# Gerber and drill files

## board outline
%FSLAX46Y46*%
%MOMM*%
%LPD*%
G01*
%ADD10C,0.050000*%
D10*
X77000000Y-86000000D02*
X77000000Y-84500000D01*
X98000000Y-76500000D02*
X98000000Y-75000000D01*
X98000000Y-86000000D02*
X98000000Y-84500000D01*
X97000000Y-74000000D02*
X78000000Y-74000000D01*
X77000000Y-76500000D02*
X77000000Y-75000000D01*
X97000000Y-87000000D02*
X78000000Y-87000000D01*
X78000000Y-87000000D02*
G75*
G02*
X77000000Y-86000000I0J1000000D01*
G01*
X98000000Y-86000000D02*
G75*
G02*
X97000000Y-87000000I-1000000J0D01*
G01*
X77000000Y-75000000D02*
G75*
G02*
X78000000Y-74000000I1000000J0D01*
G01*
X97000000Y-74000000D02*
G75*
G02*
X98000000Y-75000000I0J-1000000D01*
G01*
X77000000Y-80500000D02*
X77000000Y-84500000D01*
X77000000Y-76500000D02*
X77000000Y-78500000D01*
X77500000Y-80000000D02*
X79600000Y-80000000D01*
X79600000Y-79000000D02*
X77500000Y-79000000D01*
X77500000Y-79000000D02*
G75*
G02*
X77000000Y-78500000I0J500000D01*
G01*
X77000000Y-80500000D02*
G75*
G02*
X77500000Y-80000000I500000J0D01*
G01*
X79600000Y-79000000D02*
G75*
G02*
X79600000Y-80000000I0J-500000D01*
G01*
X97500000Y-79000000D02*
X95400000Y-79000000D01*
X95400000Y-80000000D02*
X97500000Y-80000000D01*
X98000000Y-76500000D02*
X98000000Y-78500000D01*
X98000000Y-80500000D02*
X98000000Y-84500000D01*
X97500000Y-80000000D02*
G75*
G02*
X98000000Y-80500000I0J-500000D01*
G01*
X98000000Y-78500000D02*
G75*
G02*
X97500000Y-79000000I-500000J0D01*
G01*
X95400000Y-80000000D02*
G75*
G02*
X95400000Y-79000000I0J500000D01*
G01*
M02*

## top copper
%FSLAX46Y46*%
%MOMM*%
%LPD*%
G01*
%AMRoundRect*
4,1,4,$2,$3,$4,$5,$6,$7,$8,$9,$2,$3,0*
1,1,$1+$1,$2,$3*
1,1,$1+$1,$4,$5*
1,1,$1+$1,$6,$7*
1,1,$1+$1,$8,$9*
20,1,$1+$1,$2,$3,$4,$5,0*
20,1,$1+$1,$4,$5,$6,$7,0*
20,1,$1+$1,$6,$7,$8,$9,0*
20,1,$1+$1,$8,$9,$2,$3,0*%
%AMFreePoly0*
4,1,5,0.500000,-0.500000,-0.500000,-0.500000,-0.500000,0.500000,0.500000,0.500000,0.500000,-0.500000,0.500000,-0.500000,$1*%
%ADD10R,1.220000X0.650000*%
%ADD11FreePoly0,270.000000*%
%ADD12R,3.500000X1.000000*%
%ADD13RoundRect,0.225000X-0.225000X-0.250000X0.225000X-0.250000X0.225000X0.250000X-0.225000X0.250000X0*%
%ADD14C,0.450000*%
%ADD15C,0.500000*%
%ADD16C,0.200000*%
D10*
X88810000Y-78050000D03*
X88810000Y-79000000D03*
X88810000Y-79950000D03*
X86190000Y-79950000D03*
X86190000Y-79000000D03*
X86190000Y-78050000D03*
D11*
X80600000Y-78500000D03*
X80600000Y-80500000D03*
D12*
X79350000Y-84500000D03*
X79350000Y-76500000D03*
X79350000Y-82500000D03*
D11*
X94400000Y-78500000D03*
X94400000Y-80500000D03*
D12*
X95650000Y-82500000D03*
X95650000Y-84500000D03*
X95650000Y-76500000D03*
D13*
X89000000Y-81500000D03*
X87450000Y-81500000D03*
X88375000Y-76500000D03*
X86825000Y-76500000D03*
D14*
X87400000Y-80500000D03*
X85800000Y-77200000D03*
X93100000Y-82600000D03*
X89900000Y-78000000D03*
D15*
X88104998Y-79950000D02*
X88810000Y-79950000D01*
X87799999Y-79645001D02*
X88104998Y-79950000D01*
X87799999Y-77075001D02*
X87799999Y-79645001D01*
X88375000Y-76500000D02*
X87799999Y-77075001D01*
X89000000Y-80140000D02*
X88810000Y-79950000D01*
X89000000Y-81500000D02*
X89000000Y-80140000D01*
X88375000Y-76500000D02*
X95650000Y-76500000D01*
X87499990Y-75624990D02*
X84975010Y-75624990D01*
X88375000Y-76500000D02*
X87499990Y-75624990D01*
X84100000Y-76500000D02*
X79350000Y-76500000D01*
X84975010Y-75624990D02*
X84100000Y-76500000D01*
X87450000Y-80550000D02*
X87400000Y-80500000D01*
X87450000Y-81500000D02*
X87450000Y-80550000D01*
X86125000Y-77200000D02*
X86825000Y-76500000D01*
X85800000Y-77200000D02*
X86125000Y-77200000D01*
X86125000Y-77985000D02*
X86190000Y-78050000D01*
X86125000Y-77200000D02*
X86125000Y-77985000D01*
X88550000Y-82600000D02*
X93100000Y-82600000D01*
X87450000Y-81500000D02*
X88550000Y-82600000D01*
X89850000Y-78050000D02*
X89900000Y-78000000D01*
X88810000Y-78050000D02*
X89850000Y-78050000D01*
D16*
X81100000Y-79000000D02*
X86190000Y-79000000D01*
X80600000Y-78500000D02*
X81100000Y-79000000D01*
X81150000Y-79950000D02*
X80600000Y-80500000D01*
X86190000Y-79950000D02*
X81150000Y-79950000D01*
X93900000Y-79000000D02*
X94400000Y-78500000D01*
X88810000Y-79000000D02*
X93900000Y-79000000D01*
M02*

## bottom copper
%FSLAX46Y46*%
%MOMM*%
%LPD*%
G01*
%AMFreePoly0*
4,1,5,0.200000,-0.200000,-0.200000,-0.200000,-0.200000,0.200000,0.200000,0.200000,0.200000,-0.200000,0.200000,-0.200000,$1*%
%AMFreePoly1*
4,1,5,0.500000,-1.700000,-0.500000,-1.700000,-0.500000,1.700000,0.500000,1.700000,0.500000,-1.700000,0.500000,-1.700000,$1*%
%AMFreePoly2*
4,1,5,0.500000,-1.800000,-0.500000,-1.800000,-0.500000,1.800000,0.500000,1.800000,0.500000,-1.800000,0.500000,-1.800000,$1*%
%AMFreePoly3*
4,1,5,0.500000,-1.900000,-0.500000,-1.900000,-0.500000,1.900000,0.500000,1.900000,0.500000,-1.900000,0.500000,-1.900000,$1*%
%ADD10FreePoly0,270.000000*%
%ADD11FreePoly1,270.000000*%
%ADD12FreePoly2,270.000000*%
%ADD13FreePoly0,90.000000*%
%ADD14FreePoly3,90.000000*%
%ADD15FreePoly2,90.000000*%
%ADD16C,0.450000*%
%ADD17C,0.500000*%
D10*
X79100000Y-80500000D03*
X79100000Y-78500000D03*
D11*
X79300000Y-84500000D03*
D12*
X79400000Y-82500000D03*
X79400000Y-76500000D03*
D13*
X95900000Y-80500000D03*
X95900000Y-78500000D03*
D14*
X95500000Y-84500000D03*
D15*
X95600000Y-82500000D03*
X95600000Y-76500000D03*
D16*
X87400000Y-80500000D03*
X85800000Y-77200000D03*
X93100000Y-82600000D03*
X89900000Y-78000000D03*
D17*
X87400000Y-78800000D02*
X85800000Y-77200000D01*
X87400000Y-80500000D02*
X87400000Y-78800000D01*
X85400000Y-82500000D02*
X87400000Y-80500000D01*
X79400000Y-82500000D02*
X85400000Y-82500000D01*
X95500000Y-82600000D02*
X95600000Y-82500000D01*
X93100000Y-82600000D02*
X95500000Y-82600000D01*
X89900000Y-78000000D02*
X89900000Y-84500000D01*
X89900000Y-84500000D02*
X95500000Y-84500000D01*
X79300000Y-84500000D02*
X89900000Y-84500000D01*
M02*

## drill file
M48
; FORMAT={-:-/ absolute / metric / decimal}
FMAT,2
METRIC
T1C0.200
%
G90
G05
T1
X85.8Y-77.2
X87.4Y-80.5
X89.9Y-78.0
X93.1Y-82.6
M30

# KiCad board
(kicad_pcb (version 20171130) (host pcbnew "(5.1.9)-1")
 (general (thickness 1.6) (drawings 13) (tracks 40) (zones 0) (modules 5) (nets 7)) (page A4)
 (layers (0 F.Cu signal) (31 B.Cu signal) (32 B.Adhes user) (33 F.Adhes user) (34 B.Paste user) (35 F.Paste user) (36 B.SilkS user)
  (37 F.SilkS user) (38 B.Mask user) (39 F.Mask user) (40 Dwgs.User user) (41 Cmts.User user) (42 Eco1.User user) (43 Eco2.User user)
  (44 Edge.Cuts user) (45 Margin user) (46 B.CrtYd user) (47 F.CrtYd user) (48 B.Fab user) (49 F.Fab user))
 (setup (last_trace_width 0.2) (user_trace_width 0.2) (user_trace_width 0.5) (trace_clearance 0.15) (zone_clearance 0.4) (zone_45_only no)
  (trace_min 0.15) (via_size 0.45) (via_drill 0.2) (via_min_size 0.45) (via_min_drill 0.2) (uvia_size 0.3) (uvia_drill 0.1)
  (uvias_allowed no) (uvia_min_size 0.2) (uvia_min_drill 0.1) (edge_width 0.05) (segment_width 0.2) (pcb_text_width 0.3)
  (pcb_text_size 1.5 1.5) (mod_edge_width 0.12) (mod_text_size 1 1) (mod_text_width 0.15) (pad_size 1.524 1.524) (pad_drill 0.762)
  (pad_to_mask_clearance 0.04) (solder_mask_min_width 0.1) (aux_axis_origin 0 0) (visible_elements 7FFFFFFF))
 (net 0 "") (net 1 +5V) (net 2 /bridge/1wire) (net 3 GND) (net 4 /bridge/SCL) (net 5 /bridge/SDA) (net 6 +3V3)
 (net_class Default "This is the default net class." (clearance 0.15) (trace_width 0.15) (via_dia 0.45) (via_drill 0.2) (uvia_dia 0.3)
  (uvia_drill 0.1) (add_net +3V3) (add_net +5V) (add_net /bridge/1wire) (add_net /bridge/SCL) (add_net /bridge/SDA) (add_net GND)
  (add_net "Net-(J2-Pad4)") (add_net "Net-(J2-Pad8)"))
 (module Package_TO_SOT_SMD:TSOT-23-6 (layer F.Cu) (at 87.5 79)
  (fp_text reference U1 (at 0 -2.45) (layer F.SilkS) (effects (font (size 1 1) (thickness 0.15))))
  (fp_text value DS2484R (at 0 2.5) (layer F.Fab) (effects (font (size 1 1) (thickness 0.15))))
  (pad 6 smd rect (at 1.31 -0.95) (size 1.22 0.65) (layers F.Cu F.Paste F.Mask) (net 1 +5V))
  (pad 5 smd rect (at 1.31 0) (size 1.22 0.65) (layers F.Cu F.Paste F.Mask) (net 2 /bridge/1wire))
  (pad 4 smd rect (at 1.31 0.95) (size 1.22 0.65) (layers F.Cu F.Paste F.Mask) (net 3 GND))
  (pad 3 smd rect (at -1.31 0.95) (size 1.22 0.65) (layers F.Cu F.Paste F.Mask) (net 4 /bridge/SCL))
  (pad 2 smd rect (at -1.31 0) (size 1.22 0.65) (layers F.Cu F.Paste F.Mask) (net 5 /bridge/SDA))
  (pad 1 smd rect (at -1.31 -0.95) (size 1.22 0.65) (layers F.Cu F.Paste F.Mask) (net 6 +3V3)))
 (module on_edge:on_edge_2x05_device (layer F.Cu) (at 77 80.5 270)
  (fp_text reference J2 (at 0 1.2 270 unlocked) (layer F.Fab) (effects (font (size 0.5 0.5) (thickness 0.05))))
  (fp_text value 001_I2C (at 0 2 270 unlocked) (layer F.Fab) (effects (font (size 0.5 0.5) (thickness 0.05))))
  (fp_line (start 0 0) (end 4 0) (layer Edge.Cuts) (width 0.05))
  (fp_line (start -4 0) (end -2 0) (layer Edge.Cuts) (width 0.05))
  (fp_line (start -0.5 -0.5) (end -0.5 -2.6) (layer Edge.Cuts) (width 0.05))
  (fp_line (start -1.5 -2.6) (end -1.5 -0.5) (layer Edge.Cuts) (width 0.05))
  (fp_arc (start -2 -0.5) (end -2 0) (angle -90) (layer Edge.Cuts) (width 0.05))
  (fp_arc (start 0 -0.5) (end -0.5 -0.5) (angle -90) (layer Edge.Cuts) (width 0.05))
  (fp_arc (start -1 -2.6) (end -0.5 -2.6) (angle -180) (layer Edge.Cuts) (width 0.05))
  (pad 2 smd custom (at -2 -3.6 270) (size 1 1) (layers F.Cu F.Mask) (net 5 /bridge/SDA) (zone_connect 0)
   (options (clearance outline) (anchor rect)) (primitives))
  (pad 3 smd custom (at 0 -3.6 270) (size 1 1) (layers F.Cu F.Mask) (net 4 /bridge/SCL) (zone_connect 0)
   (options (clearance outline) (anchor rect)) (primitives))
  (pad 8 smd custom (at 0 -2.1 270) (size 0.4 0.4) (layers B.Cu B.Mask) (zone_connect 0) (options (clearance outline) (anchor rect))
   (primitives))
  (pad 7 smd custom (at -2 -2.1 270) (size 0.4 0.4) (layers B.Cu B.Mask) (zone_connect 0) (options (clearance outline) (anchor rect))
   (primitives))
  (pad 10 smd custom (at 4 -2.3 270) (size 1 3.4) (layers B.Cu B.Mask) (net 1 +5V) (zone_connect 0)
   (options (clearance outline) (anchor rect)) (primitives))
  (pad 9 smd custom (at 2 -2.4 270) (size 1 3.6) (layers B.Cu B.Mask) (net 6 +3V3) (zone_connect 0)
   (options (clearance outline) (anchor rect)) (primitives))
  (pad 6 smd custom (at -4 -2.4 270) (size 1 3.6) (layers B.Cu B.Mask) (zone_connect 0) (options (clearance outline) (anchor rect))
   (primitives))
  (pad 5 smd rect (at 4 -2.35 90) (size 1 3.5) (layers F.Cu F.Mask) (zone_connect 0))
  (pad 1 smd rect (at -4 -2.35 90) (size 1 3.5) (layers F.Cu F.Mask) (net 3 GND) (zone_connect 0))
  (pad 4 smd rect (at 2 -2.35 90) (size 1 3.5) (layers F.Cu F.Mask) (zone_connect 0)))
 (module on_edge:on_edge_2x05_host (layer F.Cu) (at 98 80.5 270)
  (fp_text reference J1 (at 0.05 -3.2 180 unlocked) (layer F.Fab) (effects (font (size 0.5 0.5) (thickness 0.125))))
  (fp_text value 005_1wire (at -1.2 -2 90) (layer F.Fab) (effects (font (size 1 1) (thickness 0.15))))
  (fp_line (start -1.5 0.5) (end -1.5 2.6) (layer Edge.Cuts) (width 0.05))
  (fp_line (start -0.5 2.6) (end -0.5 0.5) (layer Edge.Cuts) (width 0.05))
  (fp_line (start -4 0) (end -2 0) (layer Edge.Cuts) (width 0.05))
  (fp_line (start 0 0) (end 4 0) (layer Edge.Cuts) (width 0.05))
  (fp_arc (start 0 0.5) (end 0 0) (angle -90) (layer Edge.Cuts) (width 0.05))
  (fp_arc (start -2 0.5) (end -1.5 0.5) (angle -90) (layer Edge.Cuts) (width 0.05))
  (fp_arc (start -1 2.6) (end -1.5 2.6) (angle -180) (layer Edge.Cuts) (width 0.05))
  (pad 2 smd custom (at -2 3.6 270) (size 1 1) (layers F.Cu F.Mask) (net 2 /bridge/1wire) (zone_connect 0)
   (options (clearance outline) (anchor rect)) (primitives))
  (pad 3 smd custom (at 0 3.6 270) (size 1 1) (layers F.Cu F.Mask) (zone_connect 0) (options (clearance outline) (anchor rect)) (primitives))
  (pad 8 smd custom (at 0 2.1 90) (size 0.4 0.4) (layers B.Cu B.Mask) (zone_connect 0) (options (clearance outline) (anchor rect))
   (primitives))
  (pad 7 smd custom (at -2 2.1 90) (size 0.4 0.4) (layers B.Cu B.Mask) (zone_connect 0) (options (clearance outline) (anchor rect))
   (primitives))
  (pad 4 smd rect (at 2 2.35 270) (size 1 3.5) (layers F.Cu F.Mask) (zone_connect 0))
  (pad 10 smd custom (at 4 2.5 90) (size 1 3.8) (layers B.Cu B.Mask) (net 1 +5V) (zone_connect 0)
   (options (clearance outline) (anchor rect)) (primitives))
  (pad 9 smd custom (at 2 2.4 90) (size 1 3.6) (layers B.Cu B.Mask) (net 6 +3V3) (zone_connect 0)
   (options (clearance outline) (anchor rect)) (primitives))
  (pad 6 smd custom (at -4 2.4 90) (size 1 3.6) (layers B.Cu B.Mask) (zone_connect 0) (options (clearance outline) (anchor rect))
   (primitives))
  (pad 5 smd rect (at 4 2.35 270) (size 1 3.5) (layers F.Cu F.Mask) (zone_connect 0))
  (pad 1 smd rect (at -4 2.35 270) (size 1 3.5) (layers F.Cu F.Mask) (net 3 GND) (zone_connect 0)))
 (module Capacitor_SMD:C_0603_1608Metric (layer F.Cu) (at 88.225 81.5)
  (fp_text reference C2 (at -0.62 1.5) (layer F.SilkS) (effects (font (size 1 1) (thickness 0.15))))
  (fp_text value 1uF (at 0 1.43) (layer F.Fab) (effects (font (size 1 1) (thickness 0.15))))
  (pad 2 smd roundrect (at 0.775 0) (size 0.9 0.95) (layers F.Cu F.Paste F.Mask) (roundrect_rratio 0.25) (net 3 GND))
  (pad 1 smd roundrect (at -0.775 0) (size 0.9 0.95) (layers F.Cu F.Paste F.Mask) (roundrect_rratio 0.25) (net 6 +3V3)))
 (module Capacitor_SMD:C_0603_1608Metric (layer F.Cu) (at 87.6 76.5)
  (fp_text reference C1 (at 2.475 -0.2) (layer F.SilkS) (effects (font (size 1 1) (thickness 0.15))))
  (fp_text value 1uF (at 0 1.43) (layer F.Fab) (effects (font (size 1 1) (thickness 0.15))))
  (pad 2 smd roundrect (at 0.775 0) (size 0.9 0.95) (layers F.Cu F.Paste F.Mask) (roundrect_rratio 0.25) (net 3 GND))
  (pad 1 smd roundrect (at -0.775 0) (size 0.9 0.95) (layers F.Cu F.Paste F.Mask) (roundrect_rratio 0.25) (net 6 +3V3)))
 (gr_line (start 77 86) (end 77 84.5) (layer Edge.Cuts) (width 0.05))
 (gr_line (start 98 76.5) (end 98 75) (layer Edge.Cuts) (width 0.05))
 (gr_line (start 98 86) (end 98 84.5) (layer Edge.Cuts) (width 0.05))
 (gr_line (start 97 74) (end 78 74) (layer Edge.Cuts) (width 0.05))
 (gr_line (start 77 76.5) (end 77 75) (layer Edge.Cuts) (width 0.05))
 (gr_line (start 97 87) (end 78 87) (layer Edge.Cuts) (width 0.05))
 (gr_arc (start 78 86) (end 77 86) (angle -90) (layer Edge.Cuts) (width 0.05))
 (gr_arc (start 97 86) (end 97 87) (angle -90) (layer Edge.Cuts) (width 0.05))
 (gr_arc (start 78 75) (end 78 74) (angle -90) (layer Edge.Cuts) (width 0.05))
 (gr_arc (start 97 75) (end 98 75) (angle -90) (layer Edge.Cuts) (width 0.05))
 (segment (start 88.104998 79.95) (end 88.81 79.95) (width 0.5) (layer F.Cu) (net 3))
 (segment (start 87.799999 79.645001) (end 88.104998 79.95) (width 0.5) (layer F.Cu) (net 3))
 (segment (start 87.799999 77.075001) (end 87.799999 79.645001) (width 0.5) (layer F.Cu) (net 3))
 (segment (start 88.375 76.5) (end 87.799999 77.075001) (width 0.5) (layer F.Cu) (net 3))
 (segment (start 89 80.14) (end 88.81 79.95) (width 0.5) (layer F.Cu) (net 3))
 (segment (start 89 81.5) (end 89 80.14) (width 0.5) (layer F.Cu) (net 3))
 (segment (start 88.375 76.5) (end 95.65 76.5) (width 0.5) (layer F.Cu) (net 3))
 (segment (start 87.49999 75.62499) (end 84.97501 75.62499) (width 0.5) (layer F.Cu) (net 3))
 (segment (start 88.375 76.5) (end 87.49999 75.62499) (width 0.5) (layer F.Cu) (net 3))
 (segment (start 84.1 76.5) (end 79.35 76.5) (width 0.5) (layer F.Cu) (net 3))
 (segment (start 84.97501 75.62499) (end 84.1 76.5) (width 0.5) (layer F.Cu) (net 3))
 (via (at 87.4 80.5) (size 0.45) (drill 0.2) (layers F.Cu B.Cu) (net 6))
 (segment (start 87.45 80.55) (end 87.4 80.5) (width 0.5) (layer F.Cu) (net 6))
 (segment (start 87.45 81.5) (end 87.45 80.55) (width 0.5) (layer F.Cu) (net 6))
 (via (at 85.8 77.2) (size 0.45) (drill 0.2) (layers F.Cu B.Cu) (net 6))
 (segment (start 87.4 78.8) (end 85.8 77.2) (width 0.5) (layer B.Cu) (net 6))
 (segment (start 87.4 80.5) (end 87.4 78.8) (width 0.5) (layer B.Cu) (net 6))
 (segment (start 86.125 77.2) (end 86.825 76.5) (width 0.5) (layer F.Cu) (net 6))
 (segment (start 85.8 77.2) (end 86.125 77.2) (width 0.5) (layer F.Cu) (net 6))
 (segment (start 86.125 77.985) (end 86.19 78.05) (width 0.5) (layer F.Cu) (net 6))
 (segment (start 86.125 77.2) (end 86.125 77.985) (width 0.5) (layer F.Cu) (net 6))
 (segment (start 85.4 82.5) (end 87.4 80.5) (width 0.5) (layer B.Cu) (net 6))
 (segment (start 79.4 82.5) (end 85.4 82.5) (width 0.5) (layer B.Cu) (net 6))
 (via (at 93.1 82.6) (size 0.45) (drill 0.2) (layers F.Cu B.Cu) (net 6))
 (segment (start 88.55 82.6) (end 93.1 82.6) (width 0.5) (layer F.Cu) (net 6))
 (segment (start 87.45 81.5) (end 88.55 82.6) (width 0.5) (layer F.Cu) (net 6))
 (segment (start 95.5 82.6) (end 95.6 82.5) (width 0.5) (layer B.Cu) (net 6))
 (segment (start 93.1 82.6) (end 95.5 82.6) (width 0.5) (layer B.Cu) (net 6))
 (via (at 89.9 78) (size 0.45) (drill 0.2) (layers F.Cu B.Cu) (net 1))
 (segment (start 89.85 78.05) (end 89.9 78) (width 0.5) (layer F.Cu) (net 1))
 (segment (start 88.81 78.05) (end 89.85 78.05) (width 0.5) (layer F.Cu) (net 1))
 (segment (start 89.9 78) (end 89.9 84.5) (width 0.5) (layer B.Cu) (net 1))
 (segment (start 89.9 84.5) (end 95.5 84.5) (width 0.5) (layer B.Cu) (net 1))
 (segment (start 79.3 84.5) (end 89.9 84.5) (width 0.5) (layer B.Cu) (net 1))
 (segment (start 81.1 79) (end 86.19 79) (width 0.2) (layer F.Cu) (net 5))
 (segment (start 80.6 78.5) (end 81.1 79) (width 0.2) (layer F.Cu) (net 5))
 (segment (start 81.15 79.95) (end 80.6 80.5) (width 0.2) (layer F.Cu) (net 4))
 (segment (start 86.19 79.95) (end 81.15 79.95) (width 0.2) (layer F.Cu) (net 4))
 (segment (start 93.9 79) (end 94.4 78.5) (width 0.2) (layer F.Cu) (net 2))
 (segment (start 88.81 79) (end 93.9 79) (width 0.2) (layer F.Cu) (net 2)))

